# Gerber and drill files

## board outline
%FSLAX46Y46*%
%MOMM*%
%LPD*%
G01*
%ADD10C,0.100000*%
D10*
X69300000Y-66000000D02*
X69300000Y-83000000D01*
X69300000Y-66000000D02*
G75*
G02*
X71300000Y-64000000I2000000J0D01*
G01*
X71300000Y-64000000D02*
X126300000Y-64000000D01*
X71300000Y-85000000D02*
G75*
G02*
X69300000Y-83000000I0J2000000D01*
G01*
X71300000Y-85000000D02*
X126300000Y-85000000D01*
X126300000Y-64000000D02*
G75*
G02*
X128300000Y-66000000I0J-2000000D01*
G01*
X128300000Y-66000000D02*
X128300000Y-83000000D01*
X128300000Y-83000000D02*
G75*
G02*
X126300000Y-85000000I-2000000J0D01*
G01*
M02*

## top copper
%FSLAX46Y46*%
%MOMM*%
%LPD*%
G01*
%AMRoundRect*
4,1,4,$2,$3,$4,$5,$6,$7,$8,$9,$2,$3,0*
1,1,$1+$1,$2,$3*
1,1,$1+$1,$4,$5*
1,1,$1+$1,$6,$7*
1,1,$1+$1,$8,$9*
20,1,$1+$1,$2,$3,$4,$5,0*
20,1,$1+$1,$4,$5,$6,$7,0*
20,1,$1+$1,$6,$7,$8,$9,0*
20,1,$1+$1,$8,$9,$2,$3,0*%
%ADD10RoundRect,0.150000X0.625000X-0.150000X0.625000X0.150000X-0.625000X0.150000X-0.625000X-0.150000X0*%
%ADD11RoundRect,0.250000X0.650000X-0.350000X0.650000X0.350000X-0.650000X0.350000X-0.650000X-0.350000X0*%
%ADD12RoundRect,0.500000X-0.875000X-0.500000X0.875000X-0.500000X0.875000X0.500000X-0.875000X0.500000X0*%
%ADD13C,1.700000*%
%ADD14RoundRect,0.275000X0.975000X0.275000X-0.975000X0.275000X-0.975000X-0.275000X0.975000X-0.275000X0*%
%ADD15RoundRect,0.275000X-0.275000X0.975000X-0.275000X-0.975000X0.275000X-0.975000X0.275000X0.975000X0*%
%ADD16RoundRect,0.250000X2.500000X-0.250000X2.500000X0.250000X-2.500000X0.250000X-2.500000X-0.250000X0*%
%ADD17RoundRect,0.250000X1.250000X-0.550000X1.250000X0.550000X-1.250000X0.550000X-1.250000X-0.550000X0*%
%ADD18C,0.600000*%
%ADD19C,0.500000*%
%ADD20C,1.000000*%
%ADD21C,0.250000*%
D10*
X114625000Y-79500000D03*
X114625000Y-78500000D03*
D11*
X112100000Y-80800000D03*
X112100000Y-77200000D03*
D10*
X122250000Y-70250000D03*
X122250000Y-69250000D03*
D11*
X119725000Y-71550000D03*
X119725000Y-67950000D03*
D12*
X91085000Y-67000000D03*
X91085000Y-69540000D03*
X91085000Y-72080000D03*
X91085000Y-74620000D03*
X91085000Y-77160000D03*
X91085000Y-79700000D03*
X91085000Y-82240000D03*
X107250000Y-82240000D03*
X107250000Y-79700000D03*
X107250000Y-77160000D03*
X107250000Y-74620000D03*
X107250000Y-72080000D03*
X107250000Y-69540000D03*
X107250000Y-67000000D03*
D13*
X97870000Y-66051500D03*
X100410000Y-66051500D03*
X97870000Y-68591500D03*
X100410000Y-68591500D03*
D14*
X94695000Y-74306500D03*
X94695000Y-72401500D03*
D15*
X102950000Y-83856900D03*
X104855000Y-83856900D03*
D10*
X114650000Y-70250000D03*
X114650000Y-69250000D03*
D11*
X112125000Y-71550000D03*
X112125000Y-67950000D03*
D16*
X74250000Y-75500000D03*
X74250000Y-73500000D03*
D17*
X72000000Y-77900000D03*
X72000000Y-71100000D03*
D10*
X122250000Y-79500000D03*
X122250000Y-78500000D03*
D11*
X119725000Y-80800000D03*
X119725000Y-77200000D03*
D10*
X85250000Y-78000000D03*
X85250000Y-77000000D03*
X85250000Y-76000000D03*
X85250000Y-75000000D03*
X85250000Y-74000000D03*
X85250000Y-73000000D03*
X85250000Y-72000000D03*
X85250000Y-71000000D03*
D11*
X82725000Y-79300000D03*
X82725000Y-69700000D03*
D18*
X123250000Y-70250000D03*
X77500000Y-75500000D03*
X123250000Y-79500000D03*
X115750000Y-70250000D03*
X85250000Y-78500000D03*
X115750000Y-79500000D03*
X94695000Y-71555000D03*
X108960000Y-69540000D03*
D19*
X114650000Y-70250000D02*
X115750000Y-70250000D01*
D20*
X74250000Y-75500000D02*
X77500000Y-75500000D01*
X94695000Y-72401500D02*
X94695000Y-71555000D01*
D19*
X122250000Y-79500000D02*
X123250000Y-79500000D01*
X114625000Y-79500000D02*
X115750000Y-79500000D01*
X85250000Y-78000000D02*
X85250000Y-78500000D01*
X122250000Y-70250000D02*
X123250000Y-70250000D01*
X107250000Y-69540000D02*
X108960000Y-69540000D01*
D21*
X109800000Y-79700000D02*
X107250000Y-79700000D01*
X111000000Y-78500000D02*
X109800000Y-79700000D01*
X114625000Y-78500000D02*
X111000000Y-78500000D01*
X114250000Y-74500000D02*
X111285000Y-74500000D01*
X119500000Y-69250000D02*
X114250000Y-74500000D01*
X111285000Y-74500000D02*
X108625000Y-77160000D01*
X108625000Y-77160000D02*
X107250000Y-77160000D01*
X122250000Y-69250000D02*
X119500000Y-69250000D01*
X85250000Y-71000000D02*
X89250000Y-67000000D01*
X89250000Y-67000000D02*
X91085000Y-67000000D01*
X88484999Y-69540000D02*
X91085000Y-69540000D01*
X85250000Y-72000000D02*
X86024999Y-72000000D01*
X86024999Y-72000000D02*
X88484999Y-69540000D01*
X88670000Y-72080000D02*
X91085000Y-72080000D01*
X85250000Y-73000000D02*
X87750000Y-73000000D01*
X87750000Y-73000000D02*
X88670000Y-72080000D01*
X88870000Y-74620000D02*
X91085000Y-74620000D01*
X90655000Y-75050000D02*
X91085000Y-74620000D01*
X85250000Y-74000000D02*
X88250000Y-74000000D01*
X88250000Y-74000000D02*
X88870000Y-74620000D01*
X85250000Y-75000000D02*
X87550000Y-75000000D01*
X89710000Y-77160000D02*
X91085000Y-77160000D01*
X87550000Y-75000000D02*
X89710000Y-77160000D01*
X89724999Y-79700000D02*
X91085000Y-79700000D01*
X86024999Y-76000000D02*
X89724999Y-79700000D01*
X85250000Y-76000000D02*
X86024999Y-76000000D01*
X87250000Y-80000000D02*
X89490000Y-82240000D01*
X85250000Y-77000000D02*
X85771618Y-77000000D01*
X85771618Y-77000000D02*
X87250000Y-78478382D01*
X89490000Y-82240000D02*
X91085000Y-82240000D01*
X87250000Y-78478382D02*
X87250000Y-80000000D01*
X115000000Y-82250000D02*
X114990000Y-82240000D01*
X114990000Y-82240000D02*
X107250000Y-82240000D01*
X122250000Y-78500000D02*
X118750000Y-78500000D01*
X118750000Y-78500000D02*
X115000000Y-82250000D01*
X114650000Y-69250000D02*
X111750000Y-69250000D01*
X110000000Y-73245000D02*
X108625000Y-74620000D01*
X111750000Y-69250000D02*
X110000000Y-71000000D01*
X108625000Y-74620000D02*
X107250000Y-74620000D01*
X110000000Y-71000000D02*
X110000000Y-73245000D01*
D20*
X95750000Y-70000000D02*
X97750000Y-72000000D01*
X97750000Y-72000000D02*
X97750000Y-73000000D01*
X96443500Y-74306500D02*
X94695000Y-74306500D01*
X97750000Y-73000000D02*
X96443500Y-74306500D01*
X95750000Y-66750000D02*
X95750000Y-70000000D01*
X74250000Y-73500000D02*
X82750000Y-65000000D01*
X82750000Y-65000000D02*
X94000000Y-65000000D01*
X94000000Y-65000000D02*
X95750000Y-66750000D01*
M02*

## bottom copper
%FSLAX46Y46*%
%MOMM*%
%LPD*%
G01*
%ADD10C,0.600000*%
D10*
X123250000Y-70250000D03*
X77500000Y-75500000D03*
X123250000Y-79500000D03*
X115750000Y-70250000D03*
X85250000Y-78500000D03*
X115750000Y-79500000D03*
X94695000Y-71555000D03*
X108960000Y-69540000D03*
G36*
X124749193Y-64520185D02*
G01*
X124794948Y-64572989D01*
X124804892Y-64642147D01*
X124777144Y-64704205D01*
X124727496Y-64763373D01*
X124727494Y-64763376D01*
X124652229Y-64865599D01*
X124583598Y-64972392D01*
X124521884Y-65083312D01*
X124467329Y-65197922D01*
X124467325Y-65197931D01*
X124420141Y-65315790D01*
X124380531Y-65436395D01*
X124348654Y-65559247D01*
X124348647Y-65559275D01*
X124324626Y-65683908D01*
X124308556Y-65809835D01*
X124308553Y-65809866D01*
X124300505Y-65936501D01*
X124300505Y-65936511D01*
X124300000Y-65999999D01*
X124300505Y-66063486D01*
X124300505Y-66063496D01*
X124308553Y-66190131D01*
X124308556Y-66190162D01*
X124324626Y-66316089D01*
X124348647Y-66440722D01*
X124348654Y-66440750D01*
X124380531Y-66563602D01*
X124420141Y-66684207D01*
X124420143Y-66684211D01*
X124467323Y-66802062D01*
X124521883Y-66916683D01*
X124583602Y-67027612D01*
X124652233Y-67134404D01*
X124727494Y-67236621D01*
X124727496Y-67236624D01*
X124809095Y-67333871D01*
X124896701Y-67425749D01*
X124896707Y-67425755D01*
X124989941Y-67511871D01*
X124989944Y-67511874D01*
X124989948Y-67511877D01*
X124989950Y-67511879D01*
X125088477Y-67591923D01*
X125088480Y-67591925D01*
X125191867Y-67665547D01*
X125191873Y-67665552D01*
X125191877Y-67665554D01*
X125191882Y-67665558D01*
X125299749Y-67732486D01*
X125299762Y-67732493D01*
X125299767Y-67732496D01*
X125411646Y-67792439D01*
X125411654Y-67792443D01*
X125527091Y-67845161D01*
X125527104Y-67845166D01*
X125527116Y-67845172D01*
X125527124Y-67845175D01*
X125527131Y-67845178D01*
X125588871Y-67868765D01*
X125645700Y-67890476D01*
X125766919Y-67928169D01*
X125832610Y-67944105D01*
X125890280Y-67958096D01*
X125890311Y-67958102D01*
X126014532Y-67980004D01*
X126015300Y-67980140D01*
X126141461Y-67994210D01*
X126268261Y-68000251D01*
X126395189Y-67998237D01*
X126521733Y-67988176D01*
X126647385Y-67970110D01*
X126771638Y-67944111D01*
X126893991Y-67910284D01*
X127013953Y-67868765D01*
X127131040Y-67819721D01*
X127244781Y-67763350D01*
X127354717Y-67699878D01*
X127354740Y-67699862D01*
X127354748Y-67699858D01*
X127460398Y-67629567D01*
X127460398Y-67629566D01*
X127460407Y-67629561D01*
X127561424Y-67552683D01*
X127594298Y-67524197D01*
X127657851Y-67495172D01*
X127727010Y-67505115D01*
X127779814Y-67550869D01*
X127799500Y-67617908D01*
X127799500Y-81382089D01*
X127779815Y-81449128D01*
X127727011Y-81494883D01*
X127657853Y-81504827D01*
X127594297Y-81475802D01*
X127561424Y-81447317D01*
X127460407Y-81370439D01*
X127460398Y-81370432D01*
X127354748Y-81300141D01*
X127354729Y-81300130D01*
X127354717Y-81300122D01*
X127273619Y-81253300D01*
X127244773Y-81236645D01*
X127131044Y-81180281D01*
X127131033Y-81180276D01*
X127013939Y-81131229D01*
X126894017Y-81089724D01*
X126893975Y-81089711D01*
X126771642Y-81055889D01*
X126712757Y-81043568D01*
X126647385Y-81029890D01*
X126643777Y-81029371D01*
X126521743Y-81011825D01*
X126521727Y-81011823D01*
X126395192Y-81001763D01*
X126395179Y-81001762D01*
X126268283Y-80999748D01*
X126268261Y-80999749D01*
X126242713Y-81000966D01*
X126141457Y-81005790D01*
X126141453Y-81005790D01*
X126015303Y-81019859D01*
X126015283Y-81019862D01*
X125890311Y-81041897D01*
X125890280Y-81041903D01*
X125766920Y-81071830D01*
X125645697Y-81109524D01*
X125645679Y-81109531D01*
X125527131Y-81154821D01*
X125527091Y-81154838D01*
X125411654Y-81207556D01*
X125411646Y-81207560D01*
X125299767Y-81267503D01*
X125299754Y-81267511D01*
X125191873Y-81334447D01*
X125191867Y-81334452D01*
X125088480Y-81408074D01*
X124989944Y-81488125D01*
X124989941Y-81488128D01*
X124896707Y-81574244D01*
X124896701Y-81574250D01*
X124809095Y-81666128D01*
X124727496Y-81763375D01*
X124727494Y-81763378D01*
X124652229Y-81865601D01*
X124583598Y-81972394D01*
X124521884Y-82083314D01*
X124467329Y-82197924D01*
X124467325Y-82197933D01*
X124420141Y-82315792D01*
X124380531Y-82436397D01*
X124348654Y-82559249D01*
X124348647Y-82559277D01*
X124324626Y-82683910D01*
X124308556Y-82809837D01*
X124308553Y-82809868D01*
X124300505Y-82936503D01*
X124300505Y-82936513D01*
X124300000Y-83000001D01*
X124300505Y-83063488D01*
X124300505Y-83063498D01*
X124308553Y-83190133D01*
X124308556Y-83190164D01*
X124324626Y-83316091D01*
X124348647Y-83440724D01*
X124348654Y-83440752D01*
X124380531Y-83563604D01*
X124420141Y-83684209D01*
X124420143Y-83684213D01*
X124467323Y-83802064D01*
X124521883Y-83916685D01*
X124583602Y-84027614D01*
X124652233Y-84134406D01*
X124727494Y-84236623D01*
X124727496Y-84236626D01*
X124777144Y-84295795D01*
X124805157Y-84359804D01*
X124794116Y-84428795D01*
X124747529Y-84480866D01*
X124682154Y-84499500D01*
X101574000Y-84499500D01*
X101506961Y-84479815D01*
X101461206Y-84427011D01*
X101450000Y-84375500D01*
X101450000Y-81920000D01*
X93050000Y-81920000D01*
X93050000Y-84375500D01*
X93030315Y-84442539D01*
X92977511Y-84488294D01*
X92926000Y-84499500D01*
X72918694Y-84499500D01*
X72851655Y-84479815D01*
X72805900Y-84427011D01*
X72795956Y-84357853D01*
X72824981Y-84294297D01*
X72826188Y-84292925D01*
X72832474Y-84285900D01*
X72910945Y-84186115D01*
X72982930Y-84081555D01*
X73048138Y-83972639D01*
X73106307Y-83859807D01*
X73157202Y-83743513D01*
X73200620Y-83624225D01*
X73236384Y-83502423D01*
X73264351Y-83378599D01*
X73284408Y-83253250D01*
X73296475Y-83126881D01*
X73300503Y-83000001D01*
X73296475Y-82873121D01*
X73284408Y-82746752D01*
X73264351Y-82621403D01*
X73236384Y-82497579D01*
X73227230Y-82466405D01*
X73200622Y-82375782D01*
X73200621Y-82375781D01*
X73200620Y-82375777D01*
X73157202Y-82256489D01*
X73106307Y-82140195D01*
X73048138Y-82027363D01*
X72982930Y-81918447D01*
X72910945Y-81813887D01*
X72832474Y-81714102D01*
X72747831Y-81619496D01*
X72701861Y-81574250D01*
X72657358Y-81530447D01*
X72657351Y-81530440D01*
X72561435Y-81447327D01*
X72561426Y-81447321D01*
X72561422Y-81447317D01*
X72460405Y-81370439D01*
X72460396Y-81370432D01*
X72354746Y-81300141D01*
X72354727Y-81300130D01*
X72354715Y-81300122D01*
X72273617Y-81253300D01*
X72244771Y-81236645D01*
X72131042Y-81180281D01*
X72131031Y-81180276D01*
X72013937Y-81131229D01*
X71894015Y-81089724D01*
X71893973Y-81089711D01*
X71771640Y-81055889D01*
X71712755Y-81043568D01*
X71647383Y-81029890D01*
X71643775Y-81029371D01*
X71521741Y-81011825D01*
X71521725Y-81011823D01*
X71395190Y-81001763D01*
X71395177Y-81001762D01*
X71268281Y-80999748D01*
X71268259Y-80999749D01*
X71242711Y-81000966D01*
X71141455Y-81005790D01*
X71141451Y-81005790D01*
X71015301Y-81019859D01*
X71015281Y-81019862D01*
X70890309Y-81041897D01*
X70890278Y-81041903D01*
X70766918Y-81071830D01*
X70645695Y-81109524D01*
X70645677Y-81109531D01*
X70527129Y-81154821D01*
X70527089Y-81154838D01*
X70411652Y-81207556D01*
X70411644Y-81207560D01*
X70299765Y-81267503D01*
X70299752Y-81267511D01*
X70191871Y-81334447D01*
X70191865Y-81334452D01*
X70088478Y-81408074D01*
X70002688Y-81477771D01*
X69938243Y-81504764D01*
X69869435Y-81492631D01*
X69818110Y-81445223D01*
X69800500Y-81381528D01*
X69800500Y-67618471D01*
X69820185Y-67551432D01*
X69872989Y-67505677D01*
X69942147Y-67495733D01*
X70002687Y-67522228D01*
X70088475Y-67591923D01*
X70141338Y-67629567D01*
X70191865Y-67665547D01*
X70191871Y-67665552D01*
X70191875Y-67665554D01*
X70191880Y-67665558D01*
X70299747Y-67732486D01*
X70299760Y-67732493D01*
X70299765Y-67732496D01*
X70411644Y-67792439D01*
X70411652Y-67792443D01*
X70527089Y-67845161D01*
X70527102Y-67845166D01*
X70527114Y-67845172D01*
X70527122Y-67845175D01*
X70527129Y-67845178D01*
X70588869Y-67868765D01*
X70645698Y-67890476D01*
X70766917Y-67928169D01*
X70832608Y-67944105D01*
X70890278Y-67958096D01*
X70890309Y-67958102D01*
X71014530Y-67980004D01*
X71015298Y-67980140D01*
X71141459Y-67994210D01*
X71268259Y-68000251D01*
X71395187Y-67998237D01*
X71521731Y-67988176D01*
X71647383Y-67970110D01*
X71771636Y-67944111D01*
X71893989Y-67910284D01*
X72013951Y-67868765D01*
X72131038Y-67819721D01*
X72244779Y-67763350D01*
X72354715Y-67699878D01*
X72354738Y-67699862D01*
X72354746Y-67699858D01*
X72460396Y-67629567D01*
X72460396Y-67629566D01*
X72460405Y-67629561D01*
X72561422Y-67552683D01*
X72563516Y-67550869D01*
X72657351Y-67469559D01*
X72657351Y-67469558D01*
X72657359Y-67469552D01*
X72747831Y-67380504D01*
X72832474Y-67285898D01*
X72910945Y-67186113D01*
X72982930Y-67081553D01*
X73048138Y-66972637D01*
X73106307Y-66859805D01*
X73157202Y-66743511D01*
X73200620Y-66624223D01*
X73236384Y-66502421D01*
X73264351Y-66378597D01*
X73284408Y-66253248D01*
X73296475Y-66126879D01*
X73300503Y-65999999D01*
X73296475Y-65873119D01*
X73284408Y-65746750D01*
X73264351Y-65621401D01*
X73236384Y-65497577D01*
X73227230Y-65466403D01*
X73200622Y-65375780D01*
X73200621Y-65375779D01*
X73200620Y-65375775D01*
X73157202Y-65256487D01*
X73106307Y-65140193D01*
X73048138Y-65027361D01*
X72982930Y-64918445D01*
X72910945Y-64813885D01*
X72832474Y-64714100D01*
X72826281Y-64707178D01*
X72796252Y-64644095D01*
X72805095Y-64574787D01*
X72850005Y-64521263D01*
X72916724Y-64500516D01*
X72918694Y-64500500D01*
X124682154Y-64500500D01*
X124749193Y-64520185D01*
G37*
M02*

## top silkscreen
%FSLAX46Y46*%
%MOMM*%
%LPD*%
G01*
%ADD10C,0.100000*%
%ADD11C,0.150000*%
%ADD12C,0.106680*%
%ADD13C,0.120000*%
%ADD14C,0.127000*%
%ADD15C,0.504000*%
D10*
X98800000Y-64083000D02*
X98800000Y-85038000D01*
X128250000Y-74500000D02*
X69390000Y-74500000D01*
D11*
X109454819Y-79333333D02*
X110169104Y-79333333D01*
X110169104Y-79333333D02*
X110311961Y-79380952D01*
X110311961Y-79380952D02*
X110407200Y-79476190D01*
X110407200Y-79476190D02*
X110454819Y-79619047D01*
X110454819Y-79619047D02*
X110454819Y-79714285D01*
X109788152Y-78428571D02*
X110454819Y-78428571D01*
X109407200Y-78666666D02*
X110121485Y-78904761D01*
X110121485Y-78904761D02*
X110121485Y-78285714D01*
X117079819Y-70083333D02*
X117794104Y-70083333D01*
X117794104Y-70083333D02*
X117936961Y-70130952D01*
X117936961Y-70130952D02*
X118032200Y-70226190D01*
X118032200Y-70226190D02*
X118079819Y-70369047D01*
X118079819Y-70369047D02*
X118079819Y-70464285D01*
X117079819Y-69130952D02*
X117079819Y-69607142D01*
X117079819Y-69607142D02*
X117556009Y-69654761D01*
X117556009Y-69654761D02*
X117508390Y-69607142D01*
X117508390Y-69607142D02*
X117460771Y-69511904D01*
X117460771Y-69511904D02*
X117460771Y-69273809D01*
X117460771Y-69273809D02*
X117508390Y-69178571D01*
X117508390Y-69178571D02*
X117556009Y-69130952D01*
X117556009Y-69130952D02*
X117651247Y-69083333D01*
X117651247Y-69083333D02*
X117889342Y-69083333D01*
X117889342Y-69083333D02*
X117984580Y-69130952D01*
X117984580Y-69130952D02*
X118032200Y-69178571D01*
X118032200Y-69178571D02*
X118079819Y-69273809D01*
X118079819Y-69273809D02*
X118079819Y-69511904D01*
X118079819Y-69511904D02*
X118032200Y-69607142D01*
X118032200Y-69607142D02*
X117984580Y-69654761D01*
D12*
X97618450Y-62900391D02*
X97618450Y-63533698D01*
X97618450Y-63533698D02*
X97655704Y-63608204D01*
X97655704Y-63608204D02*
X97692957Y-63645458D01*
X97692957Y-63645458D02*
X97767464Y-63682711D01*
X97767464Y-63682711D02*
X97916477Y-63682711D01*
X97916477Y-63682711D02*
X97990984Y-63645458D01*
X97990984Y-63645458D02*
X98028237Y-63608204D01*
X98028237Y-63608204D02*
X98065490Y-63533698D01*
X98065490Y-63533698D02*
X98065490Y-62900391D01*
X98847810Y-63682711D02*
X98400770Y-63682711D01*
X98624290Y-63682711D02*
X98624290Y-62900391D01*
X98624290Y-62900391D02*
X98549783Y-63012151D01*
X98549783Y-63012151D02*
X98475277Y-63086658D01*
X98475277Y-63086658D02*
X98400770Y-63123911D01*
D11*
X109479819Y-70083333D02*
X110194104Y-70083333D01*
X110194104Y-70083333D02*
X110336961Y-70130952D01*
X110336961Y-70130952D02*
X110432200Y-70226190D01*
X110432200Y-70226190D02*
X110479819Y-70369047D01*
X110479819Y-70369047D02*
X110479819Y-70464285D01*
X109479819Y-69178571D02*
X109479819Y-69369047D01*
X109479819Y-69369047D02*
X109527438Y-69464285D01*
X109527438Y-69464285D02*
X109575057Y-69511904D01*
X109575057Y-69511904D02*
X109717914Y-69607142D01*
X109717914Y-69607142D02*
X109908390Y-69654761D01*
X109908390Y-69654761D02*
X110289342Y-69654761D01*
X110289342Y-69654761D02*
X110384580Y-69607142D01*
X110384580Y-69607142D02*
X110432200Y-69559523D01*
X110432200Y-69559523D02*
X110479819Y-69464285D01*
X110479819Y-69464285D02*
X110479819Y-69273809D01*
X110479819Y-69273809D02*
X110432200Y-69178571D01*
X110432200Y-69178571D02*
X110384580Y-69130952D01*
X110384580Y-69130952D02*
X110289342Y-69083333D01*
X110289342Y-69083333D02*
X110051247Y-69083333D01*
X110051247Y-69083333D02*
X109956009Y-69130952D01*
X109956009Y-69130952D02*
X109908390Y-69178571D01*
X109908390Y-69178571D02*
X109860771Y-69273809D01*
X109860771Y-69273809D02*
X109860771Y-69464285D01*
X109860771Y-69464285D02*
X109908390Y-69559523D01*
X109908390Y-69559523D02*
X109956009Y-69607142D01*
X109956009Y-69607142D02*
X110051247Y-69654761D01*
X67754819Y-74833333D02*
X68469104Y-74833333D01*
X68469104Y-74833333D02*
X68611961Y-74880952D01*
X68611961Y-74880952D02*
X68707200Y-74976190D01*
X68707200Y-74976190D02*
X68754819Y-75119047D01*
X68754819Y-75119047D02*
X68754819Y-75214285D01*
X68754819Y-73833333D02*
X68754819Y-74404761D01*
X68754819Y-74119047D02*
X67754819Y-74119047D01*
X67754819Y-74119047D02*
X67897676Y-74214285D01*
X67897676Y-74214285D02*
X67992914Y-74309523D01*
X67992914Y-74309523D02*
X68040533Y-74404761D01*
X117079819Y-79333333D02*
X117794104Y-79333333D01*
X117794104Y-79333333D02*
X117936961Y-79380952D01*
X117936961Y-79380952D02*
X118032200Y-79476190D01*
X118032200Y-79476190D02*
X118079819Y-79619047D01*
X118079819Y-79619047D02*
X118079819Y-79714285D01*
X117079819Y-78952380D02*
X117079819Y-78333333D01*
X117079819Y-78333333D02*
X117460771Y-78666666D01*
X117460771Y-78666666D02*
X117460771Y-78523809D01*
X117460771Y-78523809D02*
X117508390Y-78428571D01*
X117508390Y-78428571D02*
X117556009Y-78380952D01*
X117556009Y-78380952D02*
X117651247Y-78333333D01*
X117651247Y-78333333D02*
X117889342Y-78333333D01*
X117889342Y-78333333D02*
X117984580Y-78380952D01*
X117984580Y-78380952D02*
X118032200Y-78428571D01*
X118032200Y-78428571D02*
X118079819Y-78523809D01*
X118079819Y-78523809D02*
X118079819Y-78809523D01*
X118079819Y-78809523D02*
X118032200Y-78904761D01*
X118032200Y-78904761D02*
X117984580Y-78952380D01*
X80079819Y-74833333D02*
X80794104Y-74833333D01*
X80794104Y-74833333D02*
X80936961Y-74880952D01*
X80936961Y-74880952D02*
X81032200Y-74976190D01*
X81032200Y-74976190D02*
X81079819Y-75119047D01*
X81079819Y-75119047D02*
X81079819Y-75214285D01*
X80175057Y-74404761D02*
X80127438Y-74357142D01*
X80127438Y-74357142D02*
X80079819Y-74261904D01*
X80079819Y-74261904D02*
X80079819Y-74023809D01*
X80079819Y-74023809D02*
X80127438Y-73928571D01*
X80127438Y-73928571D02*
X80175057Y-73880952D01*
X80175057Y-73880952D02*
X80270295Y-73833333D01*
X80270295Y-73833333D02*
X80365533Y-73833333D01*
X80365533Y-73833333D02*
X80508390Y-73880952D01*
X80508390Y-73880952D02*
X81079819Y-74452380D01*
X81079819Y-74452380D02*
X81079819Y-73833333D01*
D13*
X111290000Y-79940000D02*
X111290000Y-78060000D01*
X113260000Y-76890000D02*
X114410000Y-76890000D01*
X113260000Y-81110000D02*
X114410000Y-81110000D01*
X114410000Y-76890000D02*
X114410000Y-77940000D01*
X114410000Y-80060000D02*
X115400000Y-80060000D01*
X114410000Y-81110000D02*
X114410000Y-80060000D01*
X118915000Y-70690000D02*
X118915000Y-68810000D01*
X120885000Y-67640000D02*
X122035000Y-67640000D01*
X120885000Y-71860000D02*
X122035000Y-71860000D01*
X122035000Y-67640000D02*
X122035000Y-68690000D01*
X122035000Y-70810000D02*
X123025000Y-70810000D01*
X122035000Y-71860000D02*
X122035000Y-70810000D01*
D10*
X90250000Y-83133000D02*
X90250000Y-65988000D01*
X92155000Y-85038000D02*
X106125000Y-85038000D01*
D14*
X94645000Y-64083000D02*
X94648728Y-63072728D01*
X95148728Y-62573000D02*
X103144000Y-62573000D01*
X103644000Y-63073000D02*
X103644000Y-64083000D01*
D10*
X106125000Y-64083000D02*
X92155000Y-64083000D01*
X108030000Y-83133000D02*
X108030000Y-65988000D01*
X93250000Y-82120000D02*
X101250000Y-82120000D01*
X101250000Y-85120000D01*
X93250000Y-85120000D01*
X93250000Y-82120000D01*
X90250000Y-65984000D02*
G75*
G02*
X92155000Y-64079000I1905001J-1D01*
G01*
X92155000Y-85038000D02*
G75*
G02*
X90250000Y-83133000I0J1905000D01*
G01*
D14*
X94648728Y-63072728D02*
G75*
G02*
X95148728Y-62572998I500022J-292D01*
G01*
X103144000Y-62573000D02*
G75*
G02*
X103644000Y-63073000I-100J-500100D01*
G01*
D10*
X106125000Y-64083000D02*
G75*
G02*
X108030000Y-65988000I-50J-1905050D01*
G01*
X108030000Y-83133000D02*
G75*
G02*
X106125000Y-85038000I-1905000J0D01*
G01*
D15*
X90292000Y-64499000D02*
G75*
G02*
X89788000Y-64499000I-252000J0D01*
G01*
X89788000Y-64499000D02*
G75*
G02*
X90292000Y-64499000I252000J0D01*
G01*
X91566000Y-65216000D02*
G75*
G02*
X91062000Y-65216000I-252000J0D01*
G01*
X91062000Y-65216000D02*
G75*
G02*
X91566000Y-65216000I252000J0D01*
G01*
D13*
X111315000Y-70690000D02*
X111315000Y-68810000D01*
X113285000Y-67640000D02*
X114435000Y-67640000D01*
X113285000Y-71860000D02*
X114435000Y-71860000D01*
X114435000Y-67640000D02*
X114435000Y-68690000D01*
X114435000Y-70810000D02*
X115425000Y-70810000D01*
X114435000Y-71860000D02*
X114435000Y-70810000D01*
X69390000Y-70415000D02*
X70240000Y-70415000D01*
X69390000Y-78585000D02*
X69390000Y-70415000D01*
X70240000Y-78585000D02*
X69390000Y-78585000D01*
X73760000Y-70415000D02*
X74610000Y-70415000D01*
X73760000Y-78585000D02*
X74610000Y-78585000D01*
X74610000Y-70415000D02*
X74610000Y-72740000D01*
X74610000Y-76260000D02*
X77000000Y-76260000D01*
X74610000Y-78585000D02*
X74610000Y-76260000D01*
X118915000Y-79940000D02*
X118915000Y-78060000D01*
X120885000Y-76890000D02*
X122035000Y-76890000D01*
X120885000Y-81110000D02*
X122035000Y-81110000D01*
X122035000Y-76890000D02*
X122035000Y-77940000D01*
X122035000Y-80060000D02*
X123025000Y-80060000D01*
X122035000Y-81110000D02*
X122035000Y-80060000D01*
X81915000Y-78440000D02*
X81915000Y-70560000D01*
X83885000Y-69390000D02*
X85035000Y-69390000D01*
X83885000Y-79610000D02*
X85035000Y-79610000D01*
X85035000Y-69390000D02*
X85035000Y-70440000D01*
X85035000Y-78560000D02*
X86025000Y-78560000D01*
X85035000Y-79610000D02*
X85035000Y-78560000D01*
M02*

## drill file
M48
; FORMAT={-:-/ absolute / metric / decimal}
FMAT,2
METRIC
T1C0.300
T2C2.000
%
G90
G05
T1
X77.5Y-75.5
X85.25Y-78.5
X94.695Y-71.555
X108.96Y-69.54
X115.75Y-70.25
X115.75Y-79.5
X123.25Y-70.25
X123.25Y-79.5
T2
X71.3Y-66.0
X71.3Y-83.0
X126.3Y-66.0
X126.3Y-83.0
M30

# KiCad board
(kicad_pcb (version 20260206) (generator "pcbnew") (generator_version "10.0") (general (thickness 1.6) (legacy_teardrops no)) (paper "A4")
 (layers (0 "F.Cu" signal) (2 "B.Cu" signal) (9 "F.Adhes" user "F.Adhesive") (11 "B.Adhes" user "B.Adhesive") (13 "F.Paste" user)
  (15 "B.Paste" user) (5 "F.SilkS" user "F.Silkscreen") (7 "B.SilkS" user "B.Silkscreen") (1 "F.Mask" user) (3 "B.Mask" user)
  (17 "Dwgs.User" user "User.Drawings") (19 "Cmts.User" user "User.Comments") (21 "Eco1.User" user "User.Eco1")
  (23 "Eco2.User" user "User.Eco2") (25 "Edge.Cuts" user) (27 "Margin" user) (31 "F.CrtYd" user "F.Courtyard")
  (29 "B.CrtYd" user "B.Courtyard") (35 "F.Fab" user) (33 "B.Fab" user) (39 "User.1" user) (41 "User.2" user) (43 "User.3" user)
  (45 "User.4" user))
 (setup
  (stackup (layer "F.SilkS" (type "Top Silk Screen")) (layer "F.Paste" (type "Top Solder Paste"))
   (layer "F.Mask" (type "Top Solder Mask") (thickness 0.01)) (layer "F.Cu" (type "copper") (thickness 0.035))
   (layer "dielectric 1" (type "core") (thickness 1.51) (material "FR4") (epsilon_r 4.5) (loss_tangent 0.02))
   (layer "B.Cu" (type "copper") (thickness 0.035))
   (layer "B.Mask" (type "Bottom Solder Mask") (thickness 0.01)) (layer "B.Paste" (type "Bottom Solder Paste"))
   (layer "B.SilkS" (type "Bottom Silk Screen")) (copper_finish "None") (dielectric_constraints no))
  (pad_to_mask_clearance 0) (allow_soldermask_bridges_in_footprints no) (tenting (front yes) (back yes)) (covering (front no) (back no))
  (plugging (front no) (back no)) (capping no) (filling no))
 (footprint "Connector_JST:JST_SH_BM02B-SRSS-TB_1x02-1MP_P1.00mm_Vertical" (layer "F.Cu") (at 113.3 79 90)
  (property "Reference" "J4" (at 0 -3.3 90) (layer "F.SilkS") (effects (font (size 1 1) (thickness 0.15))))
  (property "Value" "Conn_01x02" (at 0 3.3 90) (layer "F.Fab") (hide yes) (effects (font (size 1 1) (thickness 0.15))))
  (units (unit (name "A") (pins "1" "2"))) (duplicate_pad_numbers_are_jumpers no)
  (fp_line (start -0.94 -2.01) (end 0.94 -2.01) (stroke (width 0.12) (type solid)) (layer "F.SilkS"))
  (fp_line (start 2.11 -0.04) (end 2.11 1.11) (stroke (width 0.12) (type solid)) (layer "F.SilkS"))
  (fp_line (start -2.11 -0.04) (end -2.11 1.11) (stroke (width 0.12) (type solid)) (layer "F.SilkS"))
  (fp_line (start 2.11 1.11) (end 1.06 1.11) (stroke (width 0.12) (type solid)) (layer "F.SilkS"))
  (fp_line (start -1.06 1.11) (end -1.06 2.1) (stroke (width 0.12) (type solid)) (layer "F.SilkS"))
  (fp_line (start -2.11 1.11) (end -1.06 1.11) (stroke (width 0.12) (type solid)) (layer "F.SilkS"))
  (pad "1" smd roundrect (at -0.5 1.325 90) (size 0.6 1.55) (layers "F.Cu" "F.Mask" "F.Paste") (roundrect_rratio 0.25) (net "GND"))
  (pad "2" smd roundrect (at 0.5 1.325 90) (size 0.6 1.55) (layers "F.Cu" "F.Mask" "F.Paste") (roundrect_rratio 0.25) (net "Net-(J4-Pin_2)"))
  (pad "MP" smd roundrect (at -1.8 -1.2 90) (size 1.2 1.8) (layers "F.Cu" "F.Mask" "F.Paste") (roundrect_rratio 0.208333))
  (pad "MP" smd roundrect (at 1.8 -1.2 90) (size 1.2 1.8) (layers "F.Cu" "F.Mask" "F.Paste") (roundrect_rratio 0.208333)))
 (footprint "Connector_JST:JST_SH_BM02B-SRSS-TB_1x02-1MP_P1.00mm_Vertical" (layer "F.Cu") (at 120.925 69.75 90)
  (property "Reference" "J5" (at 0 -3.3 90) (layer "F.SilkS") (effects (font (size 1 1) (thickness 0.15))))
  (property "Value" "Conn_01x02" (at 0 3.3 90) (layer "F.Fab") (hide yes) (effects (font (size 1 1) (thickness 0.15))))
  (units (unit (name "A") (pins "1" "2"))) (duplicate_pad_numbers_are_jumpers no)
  (fp_line (start -0.94 -2.01) (end 0.94 -2.01) (stroke (width 0.12) (type solid)) (layer "F.SilkS"))
  (fp_line (start 2.11 -0.04) (end 2.11 1.11) (stroke (width 0.12) (type solid)) (layer "F.SilkS"))
  (fp_line (start -2.11 -0.04) (end -2.11 1.11) (stroke (width 0.12) (type solid)) (layer "F.SilkS"))
  (fp_line (start 2.11 1.11) (end 1.06 1.11) (stroke (width 0.12) (type solid)) (layer "F.SilkS"))
  (fp_line (start -1.06 1.11) (end -1.06 2.1) (stroke (width 0.12) (type solid)) (layer "F.SilkS"))
  (fp_line (start -2.11 1.11) (end -1.06 1.11) (stroke (width 0.12) (type solid)) (layer "F.SilkS"))
  (pad "1" smd roundrect (at -0.5 1.325 90) (size 0.6 1.55) (layers "F.Cu" "F.Mask" "F.Paste") (roundrect_rratio 0.25) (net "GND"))
  (pad "2" smd roundrect (at 0.5 1.325 90) (size 0.6 1.55) (layers "F.Cu" "F.Mask" "F.Paste") (roundrect_rratio 0.25) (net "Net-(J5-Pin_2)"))
  (pad "MP" smd roundrect (at -1.8 -1.2 90) (size 1.2 1.8) (layers "F.Cu" "F.Mask" "F.Paste") (roundrect_rratio 0.208333))
  (pad "MP" smd roundrect (at 1.8 -1.2 90) (size 1.2 1.8) (layers "F.Cu" "F.Mask" "F.Paste") (roundrect_rratio 0.208333)))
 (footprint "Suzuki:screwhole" (layer "F.Cu") (at 126.300001 65.999999)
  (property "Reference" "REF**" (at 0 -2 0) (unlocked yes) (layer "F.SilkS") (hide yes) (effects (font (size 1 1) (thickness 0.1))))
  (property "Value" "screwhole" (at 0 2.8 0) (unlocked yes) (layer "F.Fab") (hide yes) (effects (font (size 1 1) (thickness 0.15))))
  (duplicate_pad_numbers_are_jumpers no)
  (pad "" np_thru_hole circle (at 0 0) (size 2 2) (drill 2) (layers "*.Cu" "*.Mask"))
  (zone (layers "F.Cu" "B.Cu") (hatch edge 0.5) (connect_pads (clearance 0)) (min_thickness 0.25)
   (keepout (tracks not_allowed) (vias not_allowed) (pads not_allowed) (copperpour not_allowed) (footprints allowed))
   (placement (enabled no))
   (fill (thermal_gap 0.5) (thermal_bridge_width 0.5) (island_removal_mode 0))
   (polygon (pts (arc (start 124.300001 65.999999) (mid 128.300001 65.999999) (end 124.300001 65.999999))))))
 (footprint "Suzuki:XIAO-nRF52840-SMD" (layer "F.Cu") (at 90.25 85.12)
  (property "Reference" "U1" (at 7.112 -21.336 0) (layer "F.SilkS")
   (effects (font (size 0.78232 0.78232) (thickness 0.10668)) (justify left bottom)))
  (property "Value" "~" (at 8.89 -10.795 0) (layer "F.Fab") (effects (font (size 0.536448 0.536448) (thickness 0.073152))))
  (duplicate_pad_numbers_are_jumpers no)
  (fp_line (start 0 -1.987) (end 0 -19.132) (stroke (width 0.1) (type solid)) (layer "F.SilkS"))
  (fp_line (start 1.905 -0.082) (end 15.875 -0.082) (stroke (width 0.1) (type solid)) (layer "F.SilkS"))
  (fp_line (start 4.395 -21.037) (end 4.398728 -22.047272) (stroke (width 0.127) (type solid)) (layer "F.SilkS"))
  (fp_line (start 4.898728 -22.547) (end 12.894 -22.547) (stroke (width 0.127) (type solid)) (layer "F.SilkS"))
  (fp_line (start 13.394 -22.047) (end 13.394 -21.037) (stroke (width 0.127) (type solid)) (layer "F.SilkS"))
  (fp_line (start 15.875 -21.037) (end 1.905 -21.037) (stroke (width 0.1) (type solid)) (layer "F.SilkS"))
  (fp_line (start 17.78 -1.987) (end 17.78 -19.132) (stroke (width 0.1) (type solid)) (layer "F.SilkS"))
  (fp_rect (start 3 -3) (end 11 0) (stroke (width 0.1) (type default)) (fill no) (layer "F.SilkS"))
  (fp_arc (start 0 -19.136) (mid 0.557962 -20.483038) (end 1.905 -21.041) (stroke (width 0.1) (type solid)) (layer "F.SilkS"))
  (fp_arc (start 1.905 -0.082) (mid 0.557962 -0.639962) (end 0 -1.987) (stroke (width 0.1) (type solid)) (layer "F.SilkS"))
  (fp_arc (start 4.398728 -22.047272) (mid 4.545276 -22.400644) (end 4.898728 -22.547) (stroke (width 0.127) (type default))
   (layer "F.SilkS"))
  (fp_arc (start 12.894 -22.547) (mid 13.247531 -22.400546) (end 13.394 -22.047) (stroke (width 0.127) (type default)) (layer "F.SilkS"))
  (fp_arc (start 15.875 -21.037) (mid 17.222016 -20.479031) (end 17.78 -19.132) (stroke (width 0.1) (type solid)) (layer "F.SilkS"))
  (fp_arc (start 17.78 -1.987) (mid 17.222038 -0.639961) (end 15.875 -0.082) (stroke (width 0.1) (type solid)) (layer "F.SilkS"))
  (fp_circle (center -0.21 -20.621) (end -0.21 -20.875) (stroke (width 0.5) (type solid)) (fill yes) (layer "F.SilkS"))
  (fp_circle (center 1.064 -19.904) (end 1.064 -20.158) (stroke (width 0.5) (type solid)) (fill yes) (layer "F.SilkS"))
  (pad "1" smd roundrect (at 0.835 -18.12) (size 2.75 2) (layers "F.Cu" "F.Mask" "F.Paste") (roundrect_rratio 0.25) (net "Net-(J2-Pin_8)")
   (solder_mask_margin 0.0508) (thermal_bridge_angle 45))
  (pad "2" smd roundrect (at 0.835 -15.58) (size 2.75 2) (layers "F.Cu" "F.Mask" "F.Paste") (roundrect_rratio 0.25) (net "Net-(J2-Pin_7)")
   (solder_mask_margin 0.0508) (thermal_bridge_angle 45))
  (pad "3" smd roundrect (at 0.835 -13.04) (size 2.75 2) (layers "F.Cu" "F.Mask" "F.Paste") (roundrect_rratio 0.25) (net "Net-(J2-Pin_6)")
   (solder_mask_margin 0.0508) (thermal_bridge_angle 45))
  (pad "4" smd roundrect (at 0.835 -10.5) (size 2.75 2) (layers "F.Cu" "F.Mask" "F.Paste") (roundrect_rratio 0.25) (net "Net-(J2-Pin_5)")
   (solder_mask_margin 0.0508) (thermal_bridge_angle 45))
  (pad "5" smd roundrect (at 0.835 -7.96) (size 2.75 2) (layers "F.Cu" "F.Mask" "F.Paste") (roundrect_rratio 0.25) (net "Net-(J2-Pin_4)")
   (solder_mask_margin 0.0508) (thermal_bridge_angle 45))
  (pad "6" smd roundrect (at 0.835 -5.42) (size 2.75 2) (layers "F.Cu" "F.Mask" "F.Paste") (roundrect_rratio 0.25) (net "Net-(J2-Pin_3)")
   (solder_mask_margin 0.0508) (thermal_bridge_angle 45))
  (pad "7" smd roundrect (at 0.835 -2.88) (size 2.75 2) (layers "F.Cu" "F.Mask" "F.Paste") (roundrect_rratio 0.25) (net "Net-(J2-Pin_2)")
   (solder_mask_margin 0.0508) (thermal_bridge_angle 45))
  (pad "8" smd roundrect (at 17 -2.88) (size 2.75 2) (layers "F.Cu" "F.Mask" "F.Paste") (roundrect_rratio 0.25) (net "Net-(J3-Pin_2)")
   (solder_mask_margin 0.0508) (thermal_bridge_angle 45))
  (pad "9" smd roundrect (at 17 -5.42) (size 2.75 2) (layers "F.Cu" "F.Mask" "F.Paste") (roundrect_rratio 0.25) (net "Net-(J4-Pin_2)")
   (solder_mask_margin 0.0508) (thermal_bridge_angle 45))
  (pad "10" smd roundrect (at 17 -7.96) (size 2.75 2) (layers "F.Cu" "F.Mask" "F.Paste") (roundrect_rratio 0.25) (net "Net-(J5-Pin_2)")
   (solder_mask_margin 0.0508) (thermal_bridge_angle 45))
  (pad "11" smd roundrect (at 17 -10.5) (size 2.75 2) (layers "F.Cu" "F.Mask" "F.Paste") (roundrect_rratio 0.25) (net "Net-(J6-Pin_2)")
   (solder_mask_margin 0.0508) (thermal_bridge_angle 45))
  (pad "12" smd roundrect (at 17 -13.04) (size 2.75 2) (layers "F.Cu" "F.Mask" "F.Paste") (roundrect_rratio 0.25)
   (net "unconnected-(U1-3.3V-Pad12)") (solder_mask_margin 0.0508) (thermal_bridge_angle 45))
  (pad "13" smd roundrect (at 17 -15.58) (size 2.75 2) (layers "F.Cu" "F.Mask" "F.Paste") (roundrect_rratio 0.25) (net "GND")
   (solder_mask_margin 0.0508) (thermal_bridge_angle 45))
  (pad "14" smd roundrect (at 17 -18.12) (size 2.75 2) (layers "F.Cu" "F.Mask" "F.Paste") (roundrect_rratio 0.25)
   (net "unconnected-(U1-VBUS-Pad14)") (solder_mask_margin 0.0508) (thermal_bridge_angle 45))
  (pad "15" smd circle (at 7.62 -19.0685) (size 1.7 1.7) (layers "F.Cu" "F.Mask" "F.Paste"))
  (pad "16" smd circle (at 10.16 -19.0685) (size 1.7 1.7) (layers "F.Cu" "F.Mask" "F.Paste"))
  (pad "17" smd circle (at 7.62 -16.5285) (size 1.7 1.7) (layers "F.Cu" "F.Mask" "F.Paste"))
  (pad "18" smd circle (at 10.16 -16.5285) (size 1.7 1.7) (layers "F.Cu" "F.Mask" "F.Paste"))
  (pad "19" smd roundrect (at 4.445 -10.8135 180) (size 2.5 1.1) (layers "F.Cu" "F.Mask" "F.Paste") (roundrect_rratio 0.25)
   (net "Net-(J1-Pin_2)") (thermal_bridge_angle 45))
  (pad "20" smd roundrect (at 4.445 -12.7185 180) (size 2.5 1.1) (layers "F.Cu" "F.Mask" "F.Paste") (roundrect_rratio 0.25) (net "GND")
   (thermal_bridge_angle 45))
  (pad "21" smd roundrect (at 12.7 -1.2631 270) (size 2.5 1.1) (layers "F.Cu" "F.Mask" "F.Paste") (roundrect_rratio 0.25)
   (thermal_bridge_angle 45))
  (pad "22" smd roundrect (at 14.605 -1.2631 270) (size 2.5 1.1) (layers "F.Cu" "F.Mask" "F.Paste") (roundrect_rratio 0.25)
   (thermal_bridge_angle 45))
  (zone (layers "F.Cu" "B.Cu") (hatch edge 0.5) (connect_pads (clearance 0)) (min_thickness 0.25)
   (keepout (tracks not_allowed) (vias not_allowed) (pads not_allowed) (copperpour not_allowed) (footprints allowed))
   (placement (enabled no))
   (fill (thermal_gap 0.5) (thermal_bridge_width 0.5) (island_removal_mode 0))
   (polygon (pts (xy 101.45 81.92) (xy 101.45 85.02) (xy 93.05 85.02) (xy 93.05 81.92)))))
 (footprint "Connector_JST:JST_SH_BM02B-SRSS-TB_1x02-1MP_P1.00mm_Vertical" (layer "F.Cu") (at 113.325 69.75 90)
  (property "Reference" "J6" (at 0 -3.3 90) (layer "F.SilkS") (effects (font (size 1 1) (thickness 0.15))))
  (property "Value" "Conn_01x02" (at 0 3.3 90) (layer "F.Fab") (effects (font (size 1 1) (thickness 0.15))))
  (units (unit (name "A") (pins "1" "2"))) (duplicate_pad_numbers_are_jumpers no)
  (fp_line (start -0.94 -2.01) (end 0.94 -2.01) (stroke (width 0.12) (type solid)) (layer "F.SilkS"))
  (fp_line (start 2.11 -0.04) (end 2.11 1.11) (stroke (width 0.12) (type solid)) (layer "F.SilkS"))
  (fp_line (start -2.11 -0.04) (end -2.11 1.11) (stroke (width 0.12) (type solid)) (layer "F.SilkS"))
  (fp_line (start 2.11 1.11) (end 1.06 1.11) (stroke (width 0.12) (type solid)) (layer "F.SilkS"))
  (fp_line (start -1.06 1.11) (end -1.06 2.1) (stroke (width 0.12) (type solid)) (layer "F.SilkS"))
  (fp_line (start -2.11 1.11) (end -1.06 1.11) (stroke (width 0.12) (type solid)) (layer "F.SilkS"))
  (pad "1" smd roundrect (at -0.5 1.325 90) (size 0.6 1.55) (layers "F.Cu" "F.Mask" "F.Paste") (roundrect_rratio 0.25) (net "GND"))
  (pad "2" smd roundrect (at 0.5 1.325 90) (size 0.6 1.55) (layers "F.Cu" "F.Mask" "F.Paste") (roundrect_rratio 0.25) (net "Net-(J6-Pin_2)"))
  (pad "MP" smd roundrect (at -1.8 -1.2 90) (size 1.2 1.8) (layers "F.Cu" "F.Mask" "F.Paste") (roundrect_rratio 0.208333))
  (pad "MP" smd roundrect (at 1.8 -1.2 90) (size 1.2 1.8) (layers "F.Cu" "F.Mask" "F.Paste") (roundrect_rratio 0.208333)))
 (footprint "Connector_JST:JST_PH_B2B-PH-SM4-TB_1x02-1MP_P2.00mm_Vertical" (layer "F.Cu") (at 73.75 74.5 90)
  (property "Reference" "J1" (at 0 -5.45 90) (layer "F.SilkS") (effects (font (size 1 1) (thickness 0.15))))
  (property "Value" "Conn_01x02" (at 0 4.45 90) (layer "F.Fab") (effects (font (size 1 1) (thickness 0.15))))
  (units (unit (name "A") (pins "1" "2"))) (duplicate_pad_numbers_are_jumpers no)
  (fp_line (start 4.085 -4.36) (end 4.085 -3.51) (stroke (width 0.12) (type solid)) (layer "F.SilkS"))
  (fp_line (start -4.085 -4.36) (end 4.085 -4.36) (stroke (width 0.12) (type solid)) (layer "F.SilkS"))
  (fp_line (start -4.085 -3.51) (end -4.085 -4.36) (stroke (width 0.12) (type solid)) (layer "F.SilkS"))
  (fp_line (start 4.085 0.01) (end 4.085 0.86) (stroke (width 0.12) (type solid)) (layer "F.SilkS"))
  (fp_line (start -4.085 0.01) (end -4.085 0.86) (stroke (width 0.12) (type solid)) (layer "F.SilkS"))
  (fp_line (start 4.085 0.86) (end 1.76 0.86) (stroke (width 0.12) (type solid)) (layer "F.SilkS"))
  (fp_line (start -1.76 0.86) (end -1.76 3.25) (stroke (width 0.12) (type solid)) (layer "F.SilkS"))
  (fp_line (start -4.085 0.86) (end -1.76 0.86) (stroke (width 0.12) (type solid)) (layer "F.SilkS"))
  (pad "1" smd roundrect (at -1 0.5 90) (size 1 5.5) (layers "F.Cu" "F.Mask" "F.Paste") (roundrect_rratio 0.25) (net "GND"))
  (pad "2" smd roundrect (at 1 0.5 90) (size 1 5.5) (layers "F.Cu" "F.Mask" "F.Paste") (roundrect_rratio 0.25) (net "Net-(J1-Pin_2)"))
  (pad "MP" smd roundrect (at -3.4 -1.75 90) (size 1.6 3) (layers "F.Cu" "F.Mask" "F.Paste") (roundrect_rratio 0.15625))
  (pad "MP" smd roundrect (at 3.4 -1.75 90) (size 1.6 3) (layers "F.Cu" "F.Mask" "F.Paste") (roundrect_rratio 0.15625)))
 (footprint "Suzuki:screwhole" (layer "F.Cu") (at 71.299999 83.000001)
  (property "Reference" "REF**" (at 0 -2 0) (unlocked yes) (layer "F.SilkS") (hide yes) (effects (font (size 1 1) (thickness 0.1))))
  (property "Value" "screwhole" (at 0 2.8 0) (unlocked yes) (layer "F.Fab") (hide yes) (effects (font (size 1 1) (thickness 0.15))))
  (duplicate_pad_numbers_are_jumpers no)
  (pad "" np_thru_hole circle (at 0 0) (size 2 2) (drill 2) (layers "*.Cu" "*.Mask"))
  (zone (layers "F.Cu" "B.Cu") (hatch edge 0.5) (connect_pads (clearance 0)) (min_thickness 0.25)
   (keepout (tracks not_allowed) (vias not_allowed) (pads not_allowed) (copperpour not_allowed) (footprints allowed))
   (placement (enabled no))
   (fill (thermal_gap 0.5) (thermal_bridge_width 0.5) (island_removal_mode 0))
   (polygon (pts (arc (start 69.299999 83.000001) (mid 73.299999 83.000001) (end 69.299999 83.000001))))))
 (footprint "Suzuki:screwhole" (layer "F.Cu") (at 126.300001 83.000001)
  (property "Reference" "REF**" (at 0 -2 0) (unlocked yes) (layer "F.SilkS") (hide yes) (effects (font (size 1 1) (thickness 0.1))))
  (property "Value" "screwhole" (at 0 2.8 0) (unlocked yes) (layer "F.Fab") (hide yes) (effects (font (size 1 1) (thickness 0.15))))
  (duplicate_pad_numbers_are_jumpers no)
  (pad "" np_thru_hole circle (at 0 0) (size 2 2) (drill 2) (layers "*.Cu" "*.Mask"))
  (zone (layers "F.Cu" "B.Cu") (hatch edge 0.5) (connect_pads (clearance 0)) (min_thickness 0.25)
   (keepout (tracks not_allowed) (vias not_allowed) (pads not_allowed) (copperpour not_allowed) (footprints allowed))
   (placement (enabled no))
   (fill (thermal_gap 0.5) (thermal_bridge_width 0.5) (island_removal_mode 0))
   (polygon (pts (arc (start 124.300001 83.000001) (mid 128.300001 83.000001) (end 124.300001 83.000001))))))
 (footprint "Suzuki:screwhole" (layer "F.Cu") (at 71.299999 65.999999)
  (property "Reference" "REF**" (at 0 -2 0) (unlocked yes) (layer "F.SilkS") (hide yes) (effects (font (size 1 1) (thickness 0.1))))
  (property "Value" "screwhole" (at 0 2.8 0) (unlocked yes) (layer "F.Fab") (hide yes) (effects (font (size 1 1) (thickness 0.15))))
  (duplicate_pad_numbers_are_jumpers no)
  (pad "" np_thru_hole circle (at 0 0) (size 2 2) (drill 2) (layers "*.Cu" "*.Mask"))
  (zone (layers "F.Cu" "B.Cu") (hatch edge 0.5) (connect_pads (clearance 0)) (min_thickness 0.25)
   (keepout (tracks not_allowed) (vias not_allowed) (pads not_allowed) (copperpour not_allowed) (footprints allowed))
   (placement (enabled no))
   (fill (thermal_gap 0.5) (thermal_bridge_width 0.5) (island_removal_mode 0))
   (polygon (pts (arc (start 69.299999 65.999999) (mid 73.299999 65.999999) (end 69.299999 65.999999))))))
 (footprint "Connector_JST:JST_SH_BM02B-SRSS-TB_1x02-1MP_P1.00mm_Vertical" (layer "F.Cu") (at 120.925 79 90)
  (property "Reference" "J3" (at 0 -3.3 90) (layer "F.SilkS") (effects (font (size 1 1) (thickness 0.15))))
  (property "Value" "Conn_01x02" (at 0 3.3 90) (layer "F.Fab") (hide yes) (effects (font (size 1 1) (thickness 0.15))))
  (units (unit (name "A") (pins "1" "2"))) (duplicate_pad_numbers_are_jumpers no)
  (fp_line (start -0.94 -2.01) (end 0.94 -2.01) (stroke (width 0.12) (type solid)) (layer "F.SilkS"))
  (fp_line (start 2.11 -0.04) (end 2.11 1.11) (stroke (width 0.12) (type solid)) (layer "F.SilkS"))
  (fp_line (start -2.11 -0.04) (end -2.11 1.11) (stroke (width 0.12) (type solid)) (layer "F.SilkS"))
  (fp_line (start 2.11 1.11) (end 1.06 1.11) (stroke (width 0.12) (type solid)) (layer "F.SilkS"))
  (fp_line (start -1.06 1.11) (end -1.06 2.1) (stroke (width 0.12) (type solid)) (layer "F.SilkS"))
  (fp_line (start -2.11 1.11) (end -1.06 1.11) (stroke (width 0.12) (type solid)) (layer "F.SilkS"))
  (pad "1" smd roundrect (at -0.5 1.325 90) (size 0.6 1.55) (layers "F.Cu" "F.Mask" "F.Paste") (roundrect_rratio 0.25) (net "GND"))
  (pad "2" smd roundrect (at 0.5 1.325 90) (size 0.6 1.55) (layers "F.Cu" "F.Mask" "F.Paste") (roundrect_rratio 0.25) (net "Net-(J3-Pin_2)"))
  (pad "MP" smd roundrect (at -1.8 -1.2 90) (size 1.2 1.8) (layers "F.Cu" "F.Mask" "F.Paste") (roundrect_rratio 0.208333))
  (pad "MP" smd roundrect (at 1.8 -1.2 90) (size 1.2 1.8) (layers "F.Cu" "F.Mask" "F.Paste") (roundrect_rratio 0.208333)))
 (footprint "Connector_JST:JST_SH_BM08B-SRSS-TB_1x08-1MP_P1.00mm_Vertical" (layer "F.Cu") (at 83.925 74.5 90)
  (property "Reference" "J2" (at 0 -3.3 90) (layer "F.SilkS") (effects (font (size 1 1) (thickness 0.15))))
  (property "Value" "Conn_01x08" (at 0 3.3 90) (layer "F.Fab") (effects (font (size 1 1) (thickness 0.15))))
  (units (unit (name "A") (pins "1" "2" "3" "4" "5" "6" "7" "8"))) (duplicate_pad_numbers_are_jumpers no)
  (fp_line (start -3.94 -2.01) (end 3.94 -2.01) (stroke (width 0.12) (type solid)) (layer "F.SilkS"))
  (fp_line (start 5.11 -0.04) (end 5.11 1.11) (stroke (width 0.12) (type solid)) (layer "F.SilkS"))
  (fp_line (start -5.11 -0.04) (end -5.11 1.11) (stroke (width 0.12) (type solid)) (layer "F.SilkS"))
  (fp_line (start 5.11 1.11) (end 4.06 1.11) (stroke (width 0.12) (type solid)) (layer "F.SilkS"))
  (fp_line (start -4.06 1.11) (end -4.06 2.1) (stroke (width 0.12) (type solid)) (layer "F.SilkS"))
  (fp_line (start -5.11 1.11) (end -4.06 1.11) (stroke (width 0.12) (type solid)) (layer "F.SilkS"))
  (pad "1" smd roundrect (at -3.5 1.325 90) (size 0.6 1.55) (layers "F.Cu" "F.Mask" "F.Paste") (roundrect_rratio 0.25) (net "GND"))
  (pad "2" smd roundrect (at -2.5 1.325 90) (size 0.6 1.55) (layers "F.Cu" "F.Mask" "F.Paste") (roundrect_rratio 0.25)
   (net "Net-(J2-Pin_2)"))
  (pad "3" smd roundrect (at -1.5 1.325 90) (size 0.6 1.55) (layers "F.Cu" "F.Mask" "F.Paste") (roundrect_rratio 0.25)
   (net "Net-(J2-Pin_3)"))
  (pad "4" smd roundrect (at -0.5 1.325 90) (size 0.6 1.55) (layers "F.Cu" "F.Mask" "F.Paste") (roundrect_rratio 0.25)
   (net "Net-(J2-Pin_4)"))
  (pad "5" smd roundrect (at 0.5 1.325 90) (size 0.6 1.55) (layers "F.Cu" "F.Mask" "F.Paste") (roundrect_rratio 0.25) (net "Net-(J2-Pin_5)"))
  (pad "6" smd roundrect (at 1.5 1.325 90) (size 0.6 1.55) (layers "F.Cu" "F.Mask" "F.Paste") (roundrect_rratio 0.25) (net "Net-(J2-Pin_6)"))
  (pad "7" smd roundrect (at 2.5 1.325 90) (size 0.6 1.55) (layers "F.Cu" "F.Mask" "F.Paste") (roundrect_rratio 0.25) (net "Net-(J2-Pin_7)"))
  (pad "8" smd roundrect (at 3.5 1.325 90) (size 0.6 1.55) (layers "F.Cu" "F.Mask" "F.Paste") (roundrect_rratio 0.25) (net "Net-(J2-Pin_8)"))
  (pad "MP" smd roundrect (at -4.8 -1.2 90) (size 1.2 1.8) (layers "F.Cu" "F.Mask" "F.Paste") (roundrect_rratio 0.208333))
  (pad "MP" smd roundrect (at 4.8 -1.2 90) (size 1.2 1.8) (layers "F.Cu" "F.Mask" "F.Paste") (roundrect_rratio 0.208333)))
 (gr_line (start 98.8 64.083) (end 98.8 85.038) (stroke (width 0.1) (type solid)) (layer "F.SilkS"))
 (gr_line (start 128.25 74.5) (end 69.39 74.5) (stroke (width 0.1) (type solid)) (layer "F.SilkS"))
 (gr_line (start 69.3 66) (end 69.3 83) (stroke (width 0.1) (type solid)) (layer "Edge.Cuts"))
 (gr_arc (start 69.3 66) (mid 69.885786 64.585786) (end 71.3 64) (stroke (width 0.1) (type default)) (layer "Edge.Cuts"))
 (gr_line (start 71.3 64) (end 126.3 64) (stroke (width 0.1) (type solid)) (layer "Edge.Cuts"))
 (gr_arc (start 71.3 85) (mid 69.885786 84.414214) (end 69.3 83) (stroke (width 0.1) (type default)) (layer "Edge.Cuts"))
 (gr_line (start 71.3 85) (end 126.3 85) (stroke (width 0.1) (type solid)) (layer "Edge.Cuts"))
 (gr_arc (start 126.3 64) (mid 127.714214 64.585786) (end 128.3 66) (stroke (width 0.1) (type default)) (layer "Edge.Cuts"))
 (gr_line (start 128.3 66) (end 128.3 83) (stroke (width 0.1) (type solid)) (layer "Edge.Cuts"))
 (gr_arc (start 128.3 83) (mid 127.714214 84.414214) (end 126.3 85) (stroke (width 0.1) (type default)) (layer "Edge.Cuts"))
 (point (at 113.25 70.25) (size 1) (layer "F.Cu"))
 (segment (start 114.65 70.25) (end 115.75 70.25) (width 0.5) (layer "F.Cu") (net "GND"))
 (segment (start 74.25 75.5) (end 77.5 75.5) (width 1) (layer "F.Cu") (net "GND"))
 (segment (start 94.695 72.4015) (end 94.695 71.555) (width 1) (layer "F.Cu") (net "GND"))
 (segment (start 122.25 79.5) (end 123.25 79.5) (width 0.5) (layer "F.Cu") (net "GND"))
 (segment (start 114.625 79.5) (end 115.75 79.5) (width 0.5) (layer "F.Cu") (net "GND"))
 (segment (start 85.25 78) (end 85.25 78.5) (width 0.5) (layer "F.Cu") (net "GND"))
 (segment (start 122.25 70.25) (end 123.25 70.25) (width 0.5) (layer "F.Cu") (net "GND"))
 (segment (start 107.25 69.54) (end 108.96 69.54) (width 0.5) (layer "F.Cu") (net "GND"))
 (via (at 123.25 70.25) (size 0.6) (drill 0.3) (layers "F.Cu" "B.Cu") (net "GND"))
 (via (at 77.5 75.5) (size 0.6) (drill 0.3) (layers "F.Cu" "B.Cu") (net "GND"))
 (via (at 123.25 79.5) (size 0.6) (drill 0.3) (layers "F.Cu" "B.Cu") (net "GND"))
 (via (at 115.75 70.25) (size 0.6) (drill 0.3) (layers "F.Cu" "B.Cu") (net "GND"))
 (via (at 85.25 78.5) (size 0.6) (drill 0.3) (layers "F.Cu" "B.Cu") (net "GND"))
 (via (at 115.75 79.5) (size 0.6) (drill 0.3) (layers "F.Cu" "B.Cu") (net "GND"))
 (via (at 94.695 71.555) (size 0.6) (drill 0.3) (layers "F.Cu" "B.Cu") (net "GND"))
 (via (at 108.96 69.54) (size 0.6) (drill 0.3) (layers "F.Cu" "B.Cu") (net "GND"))
 (segment (start 109.8 79.7) (end 107.25 79.7) (width 0.25) (layer "F.Cu") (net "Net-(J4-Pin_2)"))
 (segment (start 111 78.5) (end 109.8 79.7) (width 0.25) (layer "F.Cu") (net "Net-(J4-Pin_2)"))
 (segment (start 114.625 78.5) (end 111 78.5) (width 0.25) (layer "F.Cu") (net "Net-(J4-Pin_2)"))
 (segment (start 114.25 74.5) (end 111.285 74.5) (width 0.25) (layer "F.Cu") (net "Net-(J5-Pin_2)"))
 (segment (start 119.5 69.25) (end 114.25 74.5) (width 0.25) (layer "F.Cu") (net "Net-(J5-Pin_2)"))
 (segment (start 111.285 74.5) (end 108.625 77.16) (width 0.25) (layer "F.Cu") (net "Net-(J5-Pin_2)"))
 (segment (start 108.625 77.16) (end 107.25 77.16) (width 0.25) (layer "F.Cu") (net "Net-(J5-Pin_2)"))
 (segment (start 122.25 69.25) (end 119.5 69.25) (width 0.25) (layer "F.Cu") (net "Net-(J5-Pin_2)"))
 (segment (start 85.25 71) (end 89.25 67) (width 0.25) (layer "F.Cu") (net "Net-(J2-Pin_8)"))
 (segment (start 89.25 67) (end 91.085 67) (width 0.25) (layer "F.Cu") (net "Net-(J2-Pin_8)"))
 (segment (start 88.484999 69.54) (end 91.085 69.54) (width 0.25) (layer "F.Cu") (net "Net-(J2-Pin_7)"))
 (segment (start 85.25 72) (end 86.024999 72) (width 0.25) (layer "F.Cu") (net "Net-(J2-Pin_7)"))
 (segment (start 86.024999 72) (end 88.484999 69.54) (width 0.25) (layer "F.Cu") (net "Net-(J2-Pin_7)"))
 (segment (start 88.67 72.08) (end 91.085 72.08) (width 0.25) (layer "F.Cu") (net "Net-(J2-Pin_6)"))
 (segment (start 85.25 73) (end 87.75 73) (width 0.25) (layer "F.Cu") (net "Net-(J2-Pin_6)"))
 (segment (start 87.75 73) (end 88.67 72.08) (width 0.25) (layer "F.Cu") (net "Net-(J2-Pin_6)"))
 (segment (start 88.87 74.62) (end 91.085 74.62) (width 0.25) (layer "F.Cu") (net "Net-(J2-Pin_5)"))
 (segment (start 90.655 75.05) (end 91.085 74.62) (width 0.25) (layer "F.Cu") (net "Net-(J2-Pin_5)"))
 (segment (start 85.25 74) (end 88.25 74) (width 0.25) (layer "F.Cu") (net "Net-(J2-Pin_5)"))
 (segment (start 88.25 74) (end 88.87 74.62) (width 0.25) (layer "F.Cu") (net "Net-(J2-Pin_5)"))
 (segment (start 85.25 75) (end 87.55 75) (width 0.25) (layer "F.Cu") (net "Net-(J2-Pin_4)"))
 (segment (start 89.71 77.16) (end 91.085 77.16) (width 0.25) (layer "F.Cu") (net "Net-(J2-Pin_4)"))
 (segment (start 87.55 75) (end 89.71 77.16) (width 0.25) (layer "F.Cu") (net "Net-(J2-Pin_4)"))
 (segment (start 89.724999 79.7) (end 91.085 79.7) (width 0.25) (layer "F.Cu") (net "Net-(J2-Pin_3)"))
 (segment (start 86.024999 76) (end 89.724999 79.7) (width 0.25) (layer "F.Cu") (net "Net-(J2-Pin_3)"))
 (segment (start 85.25 76) (end 86.024999 76) (width 0.25) (layer "F.Cu") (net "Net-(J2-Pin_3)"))
 (segment (start 87.25 80) (end 89.49 82.24) (width 0.25) (layer "F.Cu") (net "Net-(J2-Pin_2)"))
 (segment (start 85.25 77) (end 85.771618 77) (width 0.25) (layer "F.Cu") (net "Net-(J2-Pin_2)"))
 (segment (start 85.771618 77) (end 87.25 78.478382) (width 0.25) (layer "F.Cu") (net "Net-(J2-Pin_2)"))
 (segment (start 89.49 82.24) (end 91.085 82.24) (width 0.25) (layer "F.Cu") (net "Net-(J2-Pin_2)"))
 (segment (start 87.25 78.478382) (end 87.25 80) (width 0.25) (layer "F.Cu") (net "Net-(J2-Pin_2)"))
 (segment (start 115 82.25) (end 114.99 82.24) (width 0.25) (layer "F.Cu") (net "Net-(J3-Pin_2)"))
 (segment (start 114.99 82.24) (end 107.25 82.24) (width 0.25) (layer "F.Cu") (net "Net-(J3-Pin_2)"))
 (segment (start 122.25 78.5) (end 118.75 78.5) (width 0.25) (layer "F.Cu") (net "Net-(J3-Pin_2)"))
 (segment (start 118.75 78.5) (end 115 82.25) (width 0.25) (layer "F.Cu") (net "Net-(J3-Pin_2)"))
 (segment (start 114.65 69.25) (end 111.75 69.25) (width 0.25) (layer "F.Cu") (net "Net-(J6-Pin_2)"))
 (segment (start 110 73.245) (end 108.625 74.62) (width 0.25) (layer "F.Cu") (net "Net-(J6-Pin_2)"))
 (segment (start 111.75 69.25) (end 110 71) (width 0.25) (layer "F.Cu") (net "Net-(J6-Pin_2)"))
 (segment (start 108.625 74.62) (end 107.25 74.62) (width 0.25) (layer "F.Cu") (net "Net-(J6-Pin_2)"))
 (segment (start 110 71) (end 110 73.245) (width 0.25) (layer "F.Cu") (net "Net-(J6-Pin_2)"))
 (segment (start 95.75 70) (end 97.75 72) (width 1) (layer "F.Cu") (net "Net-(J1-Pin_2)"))
 (segment (start 97.75 72) (end 97.75 73) (width 1) (layer "F.Cu") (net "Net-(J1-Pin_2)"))
 (segment (start 96.4435 74.3065) (end 94.695 74.3065) (width 1) (layer "F.Cu") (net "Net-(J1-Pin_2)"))
 (segment (start 97.75 73) (end 96.4435 74.3065) (width 1) (layer "F.Cu") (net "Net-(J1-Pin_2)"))
 (segment (start 95.75 66.75) (end 95.75 70) (width 1) (layer "F.Cu") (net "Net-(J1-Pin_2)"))
 (segment (start 74.25 73.5) (end 82.75 65) (width 1) (layer "F.Cu") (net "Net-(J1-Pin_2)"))
 (segment (start 82.75 65) (end 94 65) (width 1) (layer "F.Cu") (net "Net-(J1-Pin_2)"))
 (segment (start 94 65) (end 95.75 66.75) (width 1) (layer "F.Cu") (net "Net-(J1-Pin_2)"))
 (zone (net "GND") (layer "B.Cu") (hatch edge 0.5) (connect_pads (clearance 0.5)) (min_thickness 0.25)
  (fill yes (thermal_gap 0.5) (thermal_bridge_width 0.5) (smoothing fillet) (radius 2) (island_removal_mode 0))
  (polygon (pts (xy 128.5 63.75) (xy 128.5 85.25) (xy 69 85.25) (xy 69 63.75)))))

